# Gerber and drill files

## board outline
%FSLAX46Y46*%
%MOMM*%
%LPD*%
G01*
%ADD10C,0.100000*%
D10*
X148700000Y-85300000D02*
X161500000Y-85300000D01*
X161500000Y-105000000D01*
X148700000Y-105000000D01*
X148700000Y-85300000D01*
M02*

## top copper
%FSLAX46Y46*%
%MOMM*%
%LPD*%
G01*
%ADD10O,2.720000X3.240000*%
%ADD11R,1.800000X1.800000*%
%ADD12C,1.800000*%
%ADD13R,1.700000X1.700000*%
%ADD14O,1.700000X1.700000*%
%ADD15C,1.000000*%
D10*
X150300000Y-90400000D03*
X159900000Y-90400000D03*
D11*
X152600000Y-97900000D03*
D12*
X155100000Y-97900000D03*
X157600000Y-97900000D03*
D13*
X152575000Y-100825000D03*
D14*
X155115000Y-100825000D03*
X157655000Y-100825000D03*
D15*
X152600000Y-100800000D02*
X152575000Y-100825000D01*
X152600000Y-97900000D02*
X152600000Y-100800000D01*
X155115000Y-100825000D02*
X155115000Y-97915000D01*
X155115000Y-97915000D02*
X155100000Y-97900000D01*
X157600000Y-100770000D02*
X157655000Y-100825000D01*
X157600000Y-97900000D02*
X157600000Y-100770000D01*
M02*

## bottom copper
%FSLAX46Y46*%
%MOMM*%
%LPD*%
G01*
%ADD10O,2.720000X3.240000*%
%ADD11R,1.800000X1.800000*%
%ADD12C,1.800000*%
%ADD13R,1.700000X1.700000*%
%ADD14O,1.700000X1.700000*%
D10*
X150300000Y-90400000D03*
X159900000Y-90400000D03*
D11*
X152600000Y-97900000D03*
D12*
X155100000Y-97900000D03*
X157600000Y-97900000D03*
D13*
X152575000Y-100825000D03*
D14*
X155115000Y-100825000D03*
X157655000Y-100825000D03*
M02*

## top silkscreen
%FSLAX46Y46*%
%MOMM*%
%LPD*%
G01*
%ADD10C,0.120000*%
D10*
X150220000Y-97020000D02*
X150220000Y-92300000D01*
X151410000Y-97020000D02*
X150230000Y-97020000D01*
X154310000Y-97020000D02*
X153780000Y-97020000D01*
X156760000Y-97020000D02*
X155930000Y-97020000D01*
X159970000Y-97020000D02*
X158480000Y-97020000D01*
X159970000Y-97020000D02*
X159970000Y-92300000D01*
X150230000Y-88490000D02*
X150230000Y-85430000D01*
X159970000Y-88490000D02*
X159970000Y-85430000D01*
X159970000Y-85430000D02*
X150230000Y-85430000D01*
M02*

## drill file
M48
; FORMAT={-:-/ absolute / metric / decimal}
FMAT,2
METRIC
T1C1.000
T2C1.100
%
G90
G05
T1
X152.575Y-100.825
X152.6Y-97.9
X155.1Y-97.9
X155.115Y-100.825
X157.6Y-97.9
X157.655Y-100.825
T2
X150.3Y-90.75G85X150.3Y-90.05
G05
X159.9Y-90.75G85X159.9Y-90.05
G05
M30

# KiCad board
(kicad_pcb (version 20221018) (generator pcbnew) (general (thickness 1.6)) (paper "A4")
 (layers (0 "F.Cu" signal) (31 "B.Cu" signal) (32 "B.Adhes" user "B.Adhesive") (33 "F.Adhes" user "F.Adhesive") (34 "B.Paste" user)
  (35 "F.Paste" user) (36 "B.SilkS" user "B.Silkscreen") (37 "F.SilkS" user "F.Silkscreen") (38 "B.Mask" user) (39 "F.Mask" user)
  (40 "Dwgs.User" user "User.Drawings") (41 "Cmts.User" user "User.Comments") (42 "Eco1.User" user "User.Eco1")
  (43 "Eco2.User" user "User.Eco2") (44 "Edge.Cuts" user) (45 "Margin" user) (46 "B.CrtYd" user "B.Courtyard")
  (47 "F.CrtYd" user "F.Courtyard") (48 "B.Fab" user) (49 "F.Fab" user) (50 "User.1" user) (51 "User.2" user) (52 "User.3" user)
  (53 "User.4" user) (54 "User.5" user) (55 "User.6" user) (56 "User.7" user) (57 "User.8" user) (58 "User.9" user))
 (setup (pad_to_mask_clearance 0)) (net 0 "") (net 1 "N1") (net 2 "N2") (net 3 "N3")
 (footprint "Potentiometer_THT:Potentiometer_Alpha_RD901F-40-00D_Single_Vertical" (layer "F.Cu") (at 152.6 97.9 90)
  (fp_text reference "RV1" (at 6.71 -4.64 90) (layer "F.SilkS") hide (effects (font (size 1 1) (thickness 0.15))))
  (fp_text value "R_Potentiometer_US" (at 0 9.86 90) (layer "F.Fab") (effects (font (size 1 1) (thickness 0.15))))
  (fp_line (start 0.88 -2.38) (end 5.6 -2.38) (stroke (width 0.12) (type solid)) (layer "F.SilkS"))
  (fp_line (start 0.88 -1.19) (end 0.88 -2.37) (stroke (width 0.12) (type solid)) (layer "F.SilkS"))
  (fp_line (start 0.88 1.71) (end 0.88 1.18) (stroke (width 0.12) (type solid)) (layer "F.SilkS"))
  (fp_line (start 0.88 4.16) (end 0.88 3.33) (stroke (width 0.12) (type solid)) (layer "F.SilkS"))
  (fp_line (start 0.88 7.37) (end 0.88 5.88) (stroke (width 0.12) (type solid)) (layer "F.SilkS"))
  (fp_line (start 0.88 7.37) (end 5.6 7.37) (stroke (width 0.12) (type solid)) (layer "F.SilkS"))
  (fp_line (start 9.41 -2.37) (end 12.47 -2.37) (stroke (width 0.12) (type solid)) (layer "F.SilkS"))
  (fp_line (start 9.41 7.37) (end 12.47 7.37) (stroke (width 0.12) (type solid)) (layer "F.SilkS"))
  (fp_line (start 12.47 7.37) (end 12.47 -2.37) (stroke (width 0.12) (type solid)) (layer "F.SilkS"))
  (pad "" thru_hole oval (at 7.5 -2.3 180) (size 2.72 3.24) (drill oval 1.1 1.8) (layers "*.Cu" "*.Mask"))
  (pad "" thru_hole oval (at 7.5 7.3 180) (size 2.72 3.24) (drill oval 1.1 1.8) (layers "*.Cu" "*.Mask"))
  (pad "1" thru_hole rect (at 0 0 180) (size 1.8 1.8) (drill 1) (layers "*.Cu" "*.Mask") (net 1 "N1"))
  (pad "2" thru_hole circle (at 0 2.5 180) (size 1.8 1.8) (drill 1) (layers "*.Cu" "*.Mask") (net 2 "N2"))
  (pad "3" thru_hole circle (at 0 5 180) (size 1.8 1.8) (drill 1) (layers "*.Cu" "*.Mask") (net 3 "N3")))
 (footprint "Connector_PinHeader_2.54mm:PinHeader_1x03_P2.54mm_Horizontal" (layer "B.Cu") (at 152.575 100.825 -90)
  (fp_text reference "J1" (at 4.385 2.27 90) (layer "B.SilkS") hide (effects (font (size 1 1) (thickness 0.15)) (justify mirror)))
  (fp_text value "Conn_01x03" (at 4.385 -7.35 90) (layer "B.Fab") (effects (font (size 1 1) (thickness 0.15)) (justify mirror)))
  (pad "1" thru_hole rect (at 0 0 270) (size 1.7 1.7) (drill 1) (layers "*.Cu" "*.Mask") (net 1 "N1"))
  (pad "2" thru_hole oval (at 0 -2.54 270) (size 1.7 1.7) (drill 1) (layers "*.Cu" "*.Mask") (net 2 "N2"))
  (pad "3" thru_hole oval (at 0 -5.08 270) (size 1.7 1.7) (drill 1) (layers "*.Cu" "*.Mask") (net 3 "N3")))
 (gr_rect (start 148.7 85.3) (end 161.5 105) (stroke (width 0.1) (type default)) (fill none) (layer "Edge.Cuts"))
 (segment (start 152.6 100.8) (end 152.575 100.825) (width 1) (layer "F.Cu") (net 1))
 (segment (start 152.6 97.9) (end 152.6 100.8) (width 1) (layer "F.Cu") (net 1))
 (segment (start 155.115 100.825) (end 155.115 97.915) (width 1) (layer "F.Cu") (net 2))
 (segment (start 155.115 97.915) (end 155.1 97.9) (width 1) (layer "F.Cu") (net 2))
 (segment (start 157.6 100.77) (end 157.655 100.825) (width 1) (layer "F.Cu") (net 3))
 (segment (start 157.6 97.9) (end 157.6 100.77) (width 1) (layer "F.Cu") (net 3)))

